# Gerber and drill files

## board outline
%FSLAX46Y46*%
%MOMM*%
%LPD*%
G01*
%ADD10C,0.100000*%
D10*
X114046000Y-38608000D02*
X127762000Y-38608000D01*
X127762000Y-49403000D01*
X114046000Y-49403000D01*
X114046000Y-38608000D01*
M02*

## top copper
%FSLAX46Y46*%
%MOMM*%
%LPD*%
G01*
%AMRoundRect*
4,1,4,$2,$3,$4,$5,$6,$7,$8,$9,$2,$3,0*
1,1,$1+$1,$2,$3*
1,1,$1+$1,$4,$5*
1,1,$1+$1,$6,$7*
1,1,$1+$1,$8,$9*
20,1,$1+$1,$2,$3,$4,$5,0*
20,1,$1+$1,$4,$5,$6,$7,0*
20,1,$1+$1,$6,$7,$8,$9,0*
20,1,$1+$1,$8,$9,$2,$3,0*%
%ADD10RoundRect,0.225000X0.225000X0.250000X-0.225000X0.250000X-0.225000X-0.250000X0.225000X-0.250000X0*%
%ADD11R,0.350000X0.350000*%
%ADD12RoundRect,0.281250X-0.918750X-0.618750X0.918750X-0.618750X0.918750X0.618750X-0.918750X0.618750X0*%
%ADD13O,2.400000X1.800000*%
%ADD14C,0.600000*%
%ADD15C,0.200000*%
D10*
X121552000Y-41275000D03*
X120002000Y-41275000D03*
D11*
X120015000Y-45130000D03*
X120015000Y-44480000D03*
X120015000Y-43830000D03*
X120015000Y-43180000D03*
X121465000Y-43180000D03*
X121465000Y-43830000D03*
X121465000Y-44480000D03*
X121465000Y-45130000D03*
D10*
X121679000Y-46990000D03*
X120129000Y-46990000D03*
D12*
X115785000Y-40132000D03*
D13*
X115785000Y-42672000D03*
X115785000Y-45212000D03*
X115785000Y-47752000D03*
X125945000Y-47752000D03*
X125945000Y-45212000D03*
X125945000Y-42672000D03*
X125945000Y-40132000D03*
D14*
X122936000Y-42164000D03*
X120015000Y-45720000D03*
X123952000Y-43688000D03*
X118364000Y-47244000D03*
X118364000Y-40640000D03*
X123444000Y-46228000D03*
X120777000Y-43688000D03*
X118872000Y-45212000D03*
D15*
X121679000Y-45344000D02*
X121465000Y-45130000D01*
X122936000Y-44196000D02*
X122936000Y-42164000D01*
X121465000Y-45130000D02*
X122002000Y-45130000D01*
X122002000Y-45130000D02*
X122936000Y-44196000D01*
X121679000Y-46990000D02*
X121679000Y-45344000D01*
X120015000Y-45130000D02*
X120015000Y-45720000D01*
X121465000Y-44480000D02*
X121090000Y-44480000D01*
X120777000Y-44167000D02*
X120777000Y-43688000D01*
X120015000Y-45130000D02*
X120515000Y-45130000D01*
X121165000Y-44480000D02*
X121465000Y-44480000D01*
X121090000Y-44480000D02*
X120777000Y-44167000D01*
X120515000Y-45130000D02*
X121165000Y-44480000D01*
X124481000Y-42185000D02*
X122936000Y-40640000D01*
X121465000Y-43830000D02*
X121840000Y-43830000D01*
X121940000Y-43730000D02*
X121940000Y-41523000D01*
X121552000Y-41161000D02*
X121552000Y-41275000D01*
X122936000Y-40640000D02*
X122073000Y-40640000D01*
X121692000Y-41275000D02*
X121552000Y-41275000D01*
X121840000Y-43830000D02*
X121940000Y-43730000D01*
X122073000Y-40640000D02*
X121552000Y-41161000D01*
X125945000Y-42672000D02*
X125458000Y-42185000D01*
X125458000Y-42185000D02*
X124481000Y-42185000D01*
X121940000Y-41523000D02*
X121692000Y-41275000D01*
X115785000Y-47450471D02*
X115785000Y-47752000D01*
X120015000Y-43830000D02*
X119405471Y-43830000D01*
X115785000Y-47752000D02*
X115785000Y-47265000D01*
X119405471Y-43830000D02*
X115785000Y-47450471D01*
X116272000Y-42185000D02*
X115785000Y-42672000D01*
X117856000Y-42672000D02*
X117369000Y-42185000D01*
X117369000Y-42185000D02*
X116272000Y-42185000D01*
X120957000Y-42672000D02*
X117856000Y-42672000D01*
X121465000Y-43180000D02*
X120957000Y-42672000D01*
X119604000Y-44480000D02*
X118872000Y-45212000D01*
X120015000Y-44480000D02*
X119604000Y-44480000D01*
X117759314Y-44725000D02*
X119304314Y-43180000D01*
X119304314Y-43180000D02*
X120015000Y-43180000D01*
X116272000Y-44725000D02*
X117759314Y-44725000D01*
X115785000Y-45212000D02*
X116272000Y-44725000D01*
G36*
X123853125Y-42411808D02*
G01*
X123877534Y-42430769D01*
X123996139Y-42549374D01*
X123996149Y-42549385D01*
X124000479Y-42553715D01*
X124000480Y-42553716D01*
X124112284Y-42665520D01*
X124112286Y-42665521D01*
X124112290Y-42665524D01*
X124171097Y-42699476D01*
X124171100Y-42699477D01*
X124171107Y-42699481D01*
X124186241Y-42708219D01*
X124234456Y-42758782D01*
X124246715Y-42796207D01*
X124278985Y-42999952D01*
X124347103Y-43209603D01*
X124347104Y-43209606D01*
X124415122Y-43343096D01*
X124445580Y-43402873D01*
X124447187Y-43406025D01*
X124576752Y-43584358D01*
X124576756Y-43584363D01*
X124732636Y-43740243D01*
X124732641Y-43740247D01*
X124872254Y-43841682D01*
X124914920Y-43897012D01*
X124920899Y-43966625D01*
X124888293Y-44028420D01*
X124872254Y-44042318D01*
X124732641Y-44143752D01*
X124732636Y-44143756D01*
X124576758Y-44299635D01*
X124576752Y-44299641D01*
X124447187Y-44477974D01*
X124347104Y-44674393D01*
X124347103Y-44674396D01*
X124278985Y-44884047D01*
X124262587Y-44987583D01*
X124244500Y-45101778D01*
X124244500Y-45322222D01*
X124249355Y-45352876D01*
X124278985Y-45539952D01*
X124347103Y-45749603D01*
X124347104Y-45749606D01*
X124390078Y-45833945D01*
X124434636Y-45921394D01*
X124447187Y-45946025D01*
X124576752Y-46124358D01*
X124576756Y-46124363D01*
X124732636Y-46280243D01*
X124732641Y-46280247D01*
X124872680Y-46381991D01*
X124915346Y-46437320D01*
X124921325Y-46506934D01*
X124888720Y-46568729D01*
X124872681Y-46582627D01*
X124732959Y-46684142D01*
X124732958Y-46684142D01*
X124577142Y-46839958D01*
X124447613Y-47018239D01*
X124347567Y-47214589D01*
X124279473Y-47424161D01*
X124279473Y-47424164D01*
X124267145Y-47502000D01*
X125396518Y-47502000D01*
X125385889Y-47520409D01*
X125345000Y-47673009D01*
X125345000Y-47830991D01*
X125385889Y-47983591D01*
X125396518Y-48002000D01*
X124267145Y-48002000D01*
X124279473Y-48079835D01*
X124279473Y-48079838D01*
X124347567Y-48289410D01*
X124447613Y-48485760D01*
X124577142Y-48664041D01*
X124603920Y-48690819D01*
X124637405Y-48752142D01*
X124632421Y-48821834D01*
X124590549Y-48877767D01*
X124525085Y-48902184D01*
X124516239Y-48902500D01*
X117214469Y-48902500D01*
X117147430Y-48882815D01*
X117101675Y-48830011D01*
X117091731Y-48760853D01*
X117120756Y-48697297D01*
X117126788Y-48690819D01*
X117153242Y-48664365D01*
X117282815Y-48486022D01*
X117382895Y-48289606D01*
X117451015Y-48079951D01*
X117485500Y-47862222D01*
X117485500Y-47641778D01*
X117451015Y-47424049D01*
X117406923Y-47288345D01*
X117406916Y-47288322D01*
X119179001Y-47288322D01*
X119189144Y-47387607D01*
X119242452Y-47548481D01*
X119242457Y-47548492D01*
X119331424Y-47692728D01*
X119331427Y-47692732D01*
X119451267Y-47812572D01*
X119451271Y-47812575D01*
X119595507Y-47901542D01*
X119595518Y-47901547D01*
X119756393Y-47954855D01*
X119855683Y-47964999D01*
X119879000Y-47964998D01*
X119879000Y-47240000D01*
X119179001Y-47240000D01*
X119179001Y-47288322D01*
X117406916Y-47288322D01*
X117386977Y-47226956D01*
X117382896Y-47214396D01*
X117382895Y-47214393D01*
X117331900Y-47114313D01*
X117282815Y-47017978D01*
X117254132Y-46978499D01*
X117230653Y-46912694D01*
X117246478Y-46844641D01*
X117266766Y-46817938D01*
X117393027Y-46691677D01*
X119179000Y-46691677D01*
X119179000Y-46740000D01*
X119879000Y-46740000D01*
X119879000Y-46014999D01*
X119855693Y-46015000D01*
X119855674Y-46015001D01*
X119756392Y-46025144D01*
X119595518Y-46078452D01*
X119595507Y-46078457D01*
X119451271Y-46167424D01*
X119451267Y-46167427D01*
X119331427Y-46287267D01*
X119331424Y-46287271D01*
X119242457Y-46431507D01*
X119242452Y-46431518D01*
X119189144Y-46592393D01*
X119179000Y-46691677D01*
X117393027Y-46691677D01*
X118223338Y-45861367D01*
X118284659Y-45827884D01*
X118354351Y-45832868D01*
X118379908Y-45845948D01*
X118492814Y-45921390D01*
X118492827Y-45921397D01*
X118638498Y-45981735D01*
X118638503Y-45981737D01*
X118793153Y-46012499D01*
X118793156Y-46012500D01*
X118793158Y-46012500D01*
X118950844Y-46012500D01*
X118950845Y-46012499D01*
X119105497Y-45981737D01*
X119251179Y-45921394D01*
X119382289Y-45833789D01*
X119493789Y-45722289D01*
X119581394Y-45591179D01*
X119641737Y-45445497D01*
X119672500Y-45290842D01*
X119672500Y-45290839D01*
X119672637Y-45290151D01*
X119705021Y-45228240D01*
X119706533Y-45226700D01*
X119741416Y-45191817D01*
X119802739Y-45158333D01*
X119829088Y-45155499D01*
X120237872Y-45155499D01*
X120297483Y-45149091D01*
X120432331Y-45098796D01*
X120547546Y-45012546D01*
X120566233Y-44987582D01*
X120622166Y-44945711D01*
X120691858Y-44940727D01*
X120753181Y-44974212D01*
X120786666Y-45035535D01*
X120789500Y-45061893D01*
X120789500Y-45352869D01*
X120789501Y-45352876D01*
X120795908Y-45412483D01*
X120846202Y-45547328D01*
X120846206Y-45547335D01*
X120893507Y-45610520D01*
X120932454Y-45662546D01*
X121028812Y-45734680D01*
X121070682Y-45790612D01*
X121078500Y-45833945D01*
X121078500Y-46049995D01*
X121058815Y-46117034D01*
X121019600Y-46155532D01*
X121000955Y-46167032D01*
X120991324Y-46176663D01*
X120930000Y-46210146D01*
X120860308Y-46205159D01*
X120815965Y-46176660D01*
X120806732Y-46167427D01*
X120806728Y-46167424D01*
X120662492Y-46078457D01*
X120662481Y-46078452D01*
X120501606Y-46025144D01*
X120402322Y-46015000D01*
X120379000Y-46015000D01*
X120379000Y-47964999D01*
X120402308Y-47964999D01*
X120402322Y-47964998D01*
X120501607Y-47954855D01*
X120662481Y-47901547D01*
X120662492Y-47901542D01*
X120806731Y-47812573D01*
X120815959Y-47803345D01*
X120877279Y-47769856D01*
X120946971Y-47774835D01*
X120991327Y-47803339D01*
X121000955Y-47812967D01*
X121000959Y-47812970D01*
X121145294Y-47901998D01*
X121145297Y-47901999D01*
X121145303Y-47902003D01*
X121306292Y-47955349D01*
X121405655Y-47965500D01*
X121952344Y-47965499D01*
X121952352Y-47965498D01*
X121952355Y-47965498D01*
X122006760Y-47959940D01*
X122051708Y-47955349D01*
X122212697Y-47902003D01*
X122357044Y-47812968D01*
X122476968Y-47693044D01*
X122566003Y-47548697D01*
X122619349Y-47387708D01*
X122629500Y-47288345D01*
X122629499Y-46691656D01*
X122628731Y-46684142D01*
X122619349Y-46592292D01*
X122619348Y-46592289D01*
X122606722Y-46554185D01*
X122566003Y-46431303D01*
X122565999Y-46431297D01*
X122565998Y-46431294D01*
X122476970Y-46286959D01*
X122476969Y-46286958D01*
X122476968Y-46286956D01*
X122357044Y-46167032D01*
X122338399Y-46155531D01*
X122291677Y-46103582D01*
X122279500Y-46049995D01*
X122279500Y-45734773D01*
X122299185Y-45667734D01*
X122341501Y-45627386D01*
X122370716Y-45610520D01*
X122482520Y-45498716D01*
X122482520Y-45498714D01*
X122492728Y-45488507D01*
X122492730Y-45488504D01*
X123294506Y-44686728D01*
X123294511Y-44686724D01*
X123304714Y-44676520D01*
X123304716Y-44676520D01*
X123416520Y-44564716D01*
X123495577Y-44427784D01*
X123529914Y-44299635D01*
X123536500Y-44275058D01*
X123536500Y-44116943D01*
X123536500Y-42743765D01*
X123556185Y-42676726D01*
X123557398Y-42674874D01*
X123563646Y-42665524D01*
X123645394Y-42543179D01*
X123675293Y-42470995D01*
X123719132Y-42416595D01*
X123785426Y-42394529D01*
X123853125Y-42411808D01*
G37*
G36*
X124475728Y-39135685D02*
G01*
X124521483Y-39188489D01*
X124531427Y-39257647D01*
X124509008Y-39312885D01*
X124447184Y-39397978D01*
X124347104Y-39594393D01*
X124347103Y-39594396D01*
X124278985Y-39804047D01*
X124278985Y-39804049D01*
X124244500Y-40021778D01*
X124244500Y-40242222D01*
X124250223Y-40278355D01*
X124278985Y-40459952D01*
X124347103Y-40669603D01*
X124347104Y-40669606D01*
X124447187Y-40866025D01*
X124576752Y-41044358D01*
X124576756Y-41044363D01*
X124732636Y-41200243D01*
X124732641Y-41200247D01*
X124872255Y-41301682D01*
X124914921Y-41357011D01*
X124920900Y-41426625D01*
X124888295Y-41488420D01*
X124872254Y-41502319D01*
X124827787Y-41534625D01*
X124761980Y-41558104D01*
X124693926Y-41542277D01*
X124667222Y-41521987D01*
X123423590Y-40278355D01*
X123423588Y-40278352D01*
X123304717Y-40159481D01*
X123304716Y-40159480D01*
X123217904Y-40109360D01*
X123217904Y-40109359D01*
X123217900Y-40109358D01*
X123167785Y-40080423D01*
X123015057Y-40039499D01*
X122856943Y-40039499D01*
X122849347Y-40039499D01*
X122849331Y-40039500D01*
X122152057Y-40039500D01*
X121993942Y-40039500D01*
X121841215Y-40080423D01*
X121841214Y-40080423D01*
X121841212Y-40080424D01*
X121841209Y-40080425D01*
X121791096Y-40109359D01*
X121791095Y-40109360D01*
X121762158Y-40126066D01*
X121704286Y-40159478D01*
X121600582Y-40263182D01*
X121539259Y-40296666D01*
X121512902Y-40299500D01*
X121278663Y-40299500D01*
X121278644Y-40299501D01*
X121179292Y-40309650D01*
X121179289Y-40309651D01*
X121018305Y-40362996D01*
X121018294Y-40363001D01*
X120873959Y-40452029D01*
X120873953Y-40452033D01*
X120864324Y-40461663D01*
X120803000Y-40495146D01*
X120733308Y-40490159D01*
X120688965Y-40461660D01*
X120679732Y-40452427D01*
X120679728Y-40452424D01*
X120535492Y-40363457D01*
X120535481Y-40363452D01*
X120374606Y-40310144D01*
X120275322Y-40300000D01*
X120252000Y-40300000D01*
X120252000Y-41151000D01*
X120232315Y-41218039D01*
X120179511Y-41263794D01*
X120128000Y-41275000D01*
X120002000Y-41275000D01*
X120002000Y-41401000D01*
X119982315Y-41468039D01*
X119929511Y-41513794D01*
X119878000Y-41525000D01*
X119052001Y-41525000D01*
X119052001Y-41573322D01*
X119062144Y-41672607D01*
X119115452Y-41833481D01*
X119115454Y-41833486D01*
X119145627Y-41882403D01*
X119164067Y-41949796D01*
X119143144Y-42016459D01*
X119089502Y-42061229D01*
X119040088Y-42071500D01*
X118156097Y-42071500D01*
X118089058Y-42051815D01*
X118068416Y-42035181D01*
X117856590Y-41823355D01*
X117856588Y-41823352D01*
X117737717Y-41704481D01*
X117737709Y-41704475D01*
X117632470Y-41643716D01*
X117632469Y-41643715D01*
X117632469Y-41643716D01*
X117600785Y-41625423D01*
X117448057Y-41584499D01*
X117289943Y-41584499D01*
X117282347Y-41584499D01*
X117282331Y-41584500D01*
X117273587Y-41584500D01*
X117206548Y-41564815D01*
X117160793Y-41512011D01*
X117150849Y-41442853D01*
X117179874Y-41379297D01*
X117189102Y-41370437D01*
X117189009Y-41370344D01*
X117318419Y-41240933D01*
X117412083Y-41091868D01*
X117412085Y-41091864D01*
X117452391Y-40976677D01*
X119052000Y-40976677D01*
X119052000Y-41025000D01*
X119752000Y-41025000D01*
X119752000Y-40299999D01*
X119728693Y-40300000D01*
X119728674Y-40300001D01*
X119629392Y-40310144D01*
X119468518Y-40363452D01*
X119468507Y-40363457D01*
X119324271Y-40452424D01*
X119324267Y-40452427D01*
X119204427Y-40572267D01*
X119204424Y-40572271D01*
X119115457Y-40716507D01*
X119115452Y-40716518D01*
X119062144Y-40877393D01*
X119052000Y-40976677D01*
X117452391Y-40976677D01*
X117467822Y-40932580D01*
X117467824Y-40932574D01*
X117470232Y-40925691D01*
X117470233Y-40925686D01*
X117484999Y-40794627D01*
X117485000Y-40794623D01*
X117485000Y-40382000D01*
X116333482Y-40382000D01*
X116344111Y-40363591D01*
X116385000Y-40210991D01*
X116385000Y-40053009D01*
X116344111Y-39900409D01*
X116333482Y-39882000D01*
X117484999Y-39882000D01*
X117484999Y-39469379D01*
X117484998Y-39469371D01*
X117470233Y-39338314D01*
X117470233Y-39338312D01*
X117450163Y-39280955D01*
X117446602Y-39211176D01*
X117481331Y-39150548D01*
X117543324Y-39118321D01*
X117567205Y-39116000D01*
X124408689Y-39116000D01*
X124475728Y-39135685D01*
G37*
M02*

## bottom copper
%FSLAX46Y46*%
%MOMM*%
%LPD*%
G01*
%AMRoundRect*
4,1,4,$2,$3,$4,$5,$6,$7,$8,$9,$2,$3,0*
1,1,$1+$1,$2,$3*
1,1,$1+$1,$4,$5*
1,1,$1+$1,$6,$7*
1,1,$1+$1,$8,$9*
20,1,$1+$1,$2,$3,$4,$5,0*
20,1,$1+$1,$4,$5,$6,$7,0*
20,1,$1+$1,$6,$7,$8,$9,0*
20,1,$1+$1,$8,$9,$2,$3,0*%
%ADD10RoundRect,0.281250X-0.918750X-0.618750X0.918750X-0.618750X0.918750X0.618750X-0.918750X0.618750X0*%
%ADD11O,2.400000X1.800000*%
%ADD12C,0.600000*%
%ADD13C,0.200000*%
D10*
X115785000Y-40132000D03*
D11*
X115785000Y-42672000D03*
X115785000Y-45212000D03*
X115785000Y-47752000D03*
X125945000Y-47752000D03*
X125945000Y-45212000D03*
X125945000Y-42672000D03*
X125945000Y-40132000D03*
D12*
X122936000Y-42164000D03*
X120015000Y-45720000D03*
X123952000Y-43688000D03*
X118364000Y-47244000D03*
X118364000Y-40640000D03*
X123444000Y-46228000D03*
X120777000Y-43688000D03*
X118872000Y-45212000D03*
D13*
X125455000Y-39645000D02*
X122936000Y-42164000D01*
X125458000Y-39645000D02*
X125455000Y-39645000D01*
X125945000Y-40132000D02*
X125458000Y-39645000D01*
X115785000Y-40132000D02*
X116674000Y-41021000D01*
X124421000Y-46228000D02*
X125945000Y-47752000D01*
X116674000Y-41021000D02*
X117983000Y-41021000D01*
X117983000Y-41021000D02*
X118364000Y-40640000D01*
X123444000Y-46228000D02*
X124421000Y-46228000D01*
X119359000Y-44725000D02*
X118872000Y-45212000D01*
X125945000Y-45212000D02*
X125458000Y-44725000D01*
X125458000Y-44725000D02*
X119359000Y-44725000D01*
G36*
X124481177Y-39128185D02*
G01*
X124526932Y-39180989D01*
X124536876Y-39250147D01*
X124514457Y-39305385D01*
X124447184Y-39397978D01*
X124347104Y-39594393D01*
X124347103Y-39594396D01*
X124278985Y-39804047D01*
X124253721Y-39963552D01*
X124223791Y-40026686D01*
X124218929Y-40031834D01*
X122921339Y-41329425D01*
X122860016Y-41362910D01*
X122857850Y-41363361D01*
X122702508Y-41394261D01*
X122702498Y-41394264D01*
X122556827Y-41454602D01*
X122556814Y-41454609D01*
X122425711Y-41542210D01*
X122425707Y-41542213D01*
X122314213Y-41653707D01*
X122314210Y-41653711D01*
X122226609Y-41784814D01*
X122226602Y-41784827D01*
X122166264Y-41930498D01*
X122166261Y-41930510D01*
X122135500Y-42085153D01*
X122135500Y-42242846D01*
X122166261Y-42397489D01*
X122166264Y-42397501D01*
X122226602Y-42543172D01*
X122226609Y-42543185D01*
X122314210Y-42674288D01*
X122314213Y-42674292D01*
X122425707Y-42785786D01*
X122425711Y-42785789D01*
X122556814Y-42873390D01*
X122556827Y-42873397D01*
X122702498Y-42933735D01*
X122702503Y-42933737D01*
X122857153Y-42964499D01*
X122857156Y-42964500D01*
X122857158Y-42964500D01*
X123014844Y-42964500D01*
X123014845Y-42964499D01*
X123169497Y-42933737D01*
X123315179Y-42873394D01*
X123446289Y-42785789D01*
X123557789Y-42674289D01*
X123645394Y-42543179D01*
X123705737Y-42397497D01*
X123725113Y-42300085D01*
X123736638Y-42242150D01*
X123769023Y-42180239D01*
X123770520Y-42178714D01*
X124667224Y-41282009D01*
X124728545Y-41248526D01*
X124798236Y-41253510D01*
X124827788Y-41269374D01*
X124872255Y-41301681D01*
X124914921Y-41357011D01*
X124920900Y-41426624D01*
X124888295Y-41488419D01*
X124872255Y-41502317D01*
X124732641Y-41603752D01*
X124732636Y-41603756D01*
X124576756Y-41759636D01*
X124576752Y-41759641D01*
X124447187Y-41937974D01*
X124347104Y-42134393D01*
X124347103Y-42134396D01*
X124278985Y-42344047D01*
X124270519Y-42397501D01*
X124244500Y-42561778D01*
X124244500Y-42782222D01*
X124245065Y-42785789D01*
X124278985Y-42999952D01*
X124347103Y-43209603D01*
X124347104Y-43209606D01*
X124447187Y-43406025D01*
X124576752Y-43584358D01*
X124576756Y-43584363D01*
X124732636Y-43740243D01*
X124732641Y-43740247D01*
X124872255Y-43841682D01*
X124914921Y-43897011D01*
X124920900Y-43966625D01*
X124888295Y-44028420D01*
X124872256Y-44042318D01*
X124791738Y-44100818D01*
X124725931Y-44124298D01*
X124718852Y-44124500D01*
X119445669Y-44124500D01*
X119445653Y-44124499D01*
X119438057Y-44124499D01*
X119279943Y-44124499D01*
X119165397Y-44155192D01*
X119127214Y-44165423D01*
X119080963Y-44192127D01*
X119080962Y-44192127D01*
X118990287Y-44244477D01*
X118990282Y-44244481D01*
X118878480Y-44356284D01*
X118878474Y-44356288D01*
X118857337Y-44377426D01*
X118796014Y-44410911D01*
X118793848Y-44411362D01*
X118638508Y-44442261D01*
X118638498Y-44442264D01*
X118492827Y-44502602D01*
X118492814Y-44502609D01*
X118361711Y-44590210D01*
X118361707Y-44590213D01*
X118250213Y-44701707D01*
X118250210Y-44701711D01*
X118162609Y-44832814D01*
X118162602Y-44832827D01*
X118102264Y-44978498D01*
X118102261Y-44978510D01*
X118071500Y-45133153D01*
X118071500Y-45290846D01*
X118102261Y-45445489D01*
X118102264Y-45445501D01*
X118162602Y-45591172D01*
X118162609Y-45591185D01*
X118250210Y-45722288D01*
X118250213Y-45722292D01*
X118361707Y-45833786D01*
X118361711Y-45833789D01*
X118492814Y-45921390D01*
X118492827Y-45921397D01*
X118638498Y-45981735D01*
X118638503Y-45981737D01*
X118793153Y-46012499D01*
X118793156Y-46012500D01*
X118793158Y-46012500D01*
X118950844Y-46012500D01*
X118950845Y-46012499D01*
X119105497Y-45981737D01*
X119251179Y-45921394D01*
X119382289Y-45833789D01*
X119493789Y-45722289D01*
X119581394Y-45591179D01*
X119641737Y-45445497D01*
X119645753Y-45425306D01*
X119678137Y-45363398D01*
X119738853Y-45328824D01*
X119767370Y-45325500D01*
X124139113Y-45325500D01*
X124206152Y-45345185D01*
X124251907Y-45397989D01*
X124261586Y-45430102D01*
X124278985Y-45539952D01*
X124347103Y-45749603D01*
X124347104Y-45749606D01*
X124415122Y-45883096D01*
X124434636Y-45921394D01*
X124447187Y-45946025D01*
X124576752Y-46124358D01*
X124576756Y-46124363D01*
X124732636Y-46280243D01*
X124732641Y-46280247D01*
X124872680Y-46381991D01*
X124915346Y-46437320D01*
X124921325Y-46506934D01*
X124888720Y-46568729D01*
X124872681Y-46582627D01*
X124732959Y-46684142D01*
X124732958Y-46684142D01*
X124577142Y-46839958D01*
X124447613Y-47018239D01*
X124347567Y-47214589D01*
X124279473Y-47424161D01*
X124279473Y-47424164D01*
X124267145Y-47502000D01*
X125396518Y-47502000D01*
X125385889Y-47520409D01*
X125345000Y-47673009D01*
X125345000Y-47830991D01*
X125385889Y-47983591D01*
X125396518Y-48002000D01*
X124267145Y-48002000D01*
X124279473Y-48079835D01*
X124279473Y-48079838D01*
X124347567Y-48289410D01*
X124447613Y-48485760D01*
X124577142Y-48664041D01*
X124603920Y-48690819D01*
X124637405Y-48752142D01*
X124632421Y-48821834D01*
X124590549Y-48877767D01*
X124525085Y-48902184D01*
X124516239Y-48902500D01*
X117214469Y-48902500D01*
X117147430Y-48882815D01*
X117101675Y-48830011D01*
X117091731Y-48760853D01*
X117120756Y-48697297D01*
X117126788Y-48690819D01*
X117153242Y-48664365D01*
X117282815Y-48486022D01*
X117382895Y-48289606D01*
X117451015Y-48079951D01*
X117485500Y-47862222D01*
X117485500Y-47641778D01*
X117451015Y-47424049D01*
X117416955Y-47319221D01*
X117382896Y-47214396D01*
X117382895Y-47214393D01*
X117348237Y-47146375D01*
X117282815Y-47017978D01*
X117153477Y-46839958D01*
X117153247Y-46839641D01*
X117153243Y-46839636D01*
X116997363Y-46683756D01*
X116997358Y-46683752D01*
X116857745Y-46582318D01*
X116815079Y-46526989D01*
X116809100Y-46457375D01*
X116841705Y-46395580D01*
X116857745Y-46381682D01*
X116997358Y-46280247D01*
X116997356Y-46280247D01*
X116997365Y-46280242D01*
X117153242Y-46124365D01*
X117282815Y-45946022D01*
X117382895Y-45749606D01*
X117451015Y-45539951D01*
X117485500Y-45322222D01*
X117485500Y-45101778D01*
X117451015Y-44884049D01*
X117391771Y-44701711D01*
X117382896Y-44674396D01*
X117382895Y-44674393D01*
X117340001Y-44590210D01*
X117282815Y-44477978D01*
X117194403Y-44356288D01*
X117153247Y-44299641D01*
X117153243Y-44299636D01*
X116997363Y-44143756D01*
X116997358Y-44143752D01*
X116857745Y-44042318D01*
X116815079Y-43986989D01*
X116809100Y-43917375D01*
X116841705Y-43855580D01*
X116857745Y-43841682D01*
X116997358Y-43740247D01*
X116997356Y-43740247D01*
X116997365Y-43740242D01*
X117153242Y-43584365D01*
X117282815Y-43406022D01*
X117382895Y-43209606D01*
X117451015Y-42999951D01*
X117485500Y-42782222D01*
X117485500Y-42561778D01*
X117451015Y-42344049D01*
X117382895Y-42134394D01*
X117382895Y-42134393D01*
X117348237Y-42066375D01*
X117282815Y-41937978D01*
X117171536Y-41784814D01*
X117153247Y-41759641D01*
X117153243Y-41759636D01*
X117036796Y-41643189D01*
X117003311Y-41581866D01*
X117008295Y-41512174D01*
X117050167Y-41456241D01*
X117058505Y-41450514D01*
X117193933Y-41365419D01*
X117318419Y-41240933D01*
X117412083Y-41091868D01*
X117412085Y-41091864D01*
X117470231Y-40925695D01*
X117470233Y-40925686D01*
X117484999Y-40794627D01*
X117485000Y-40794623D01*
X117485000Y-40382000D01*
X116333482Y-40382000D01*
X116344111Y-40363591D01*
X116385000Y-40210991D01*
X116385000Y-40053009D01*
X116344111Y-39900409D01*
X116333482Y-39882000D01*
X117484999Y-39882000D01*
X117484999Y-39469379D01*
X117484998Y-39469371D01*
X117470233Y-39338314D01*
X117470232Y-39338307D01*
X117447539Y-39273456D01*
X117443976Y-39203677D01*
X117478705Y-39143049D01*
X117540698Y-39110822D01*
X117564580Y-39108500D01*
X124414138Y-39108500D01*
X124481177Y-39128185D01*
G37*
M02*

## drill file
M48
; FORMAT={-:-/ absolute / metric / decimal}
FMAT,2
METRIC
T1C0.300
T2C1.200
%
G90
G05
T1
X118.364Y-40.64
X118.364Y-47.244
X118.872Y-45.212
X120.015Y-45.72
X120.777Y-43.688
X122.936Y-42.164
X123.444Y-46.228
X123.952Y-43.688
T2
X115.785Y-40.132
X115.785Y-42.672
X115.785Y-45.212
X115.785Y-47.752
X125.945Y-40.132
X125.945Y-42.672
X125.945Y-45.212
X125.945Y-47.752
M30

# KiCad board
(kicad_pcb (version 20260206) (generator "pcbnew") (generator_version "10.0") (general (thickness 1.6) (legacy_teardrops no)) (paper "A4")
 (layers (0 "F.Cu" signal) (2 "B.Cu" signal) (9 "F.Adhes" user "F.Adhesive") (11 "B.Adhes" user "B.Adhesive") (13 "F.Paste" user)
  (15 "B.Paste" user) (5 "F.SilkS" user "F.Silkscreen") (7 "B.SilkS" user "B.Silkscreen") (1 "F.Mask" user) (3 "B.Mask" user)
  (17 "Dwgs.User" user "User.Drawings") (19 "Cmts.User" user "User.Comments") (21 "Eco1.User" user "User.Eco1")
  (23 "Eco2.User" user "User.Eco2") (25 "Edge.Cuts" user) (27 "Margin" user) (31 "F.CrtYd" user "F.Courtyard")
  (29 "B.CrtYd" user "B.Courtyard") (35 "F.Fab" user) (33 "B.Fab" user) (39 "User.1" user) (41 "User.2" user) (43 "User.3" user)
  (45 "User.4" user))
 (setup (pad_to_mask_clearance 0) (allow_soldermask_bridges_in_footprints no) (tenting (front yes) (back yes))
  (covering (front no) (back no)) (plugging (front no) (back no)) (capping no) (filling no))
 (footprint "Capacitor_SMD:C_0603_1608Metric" (layer "F.Cu") (at 120.777 41.275 180)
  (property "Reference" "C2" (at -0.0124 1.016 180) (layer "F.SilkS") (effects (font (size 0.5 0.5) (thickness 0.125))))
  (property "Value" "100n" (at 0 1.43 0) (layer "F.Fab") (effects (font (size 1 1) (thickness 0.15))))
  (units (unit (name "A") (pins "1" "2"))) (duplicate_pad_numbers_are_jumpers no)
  (pad "1" smd roundrect (at -0.775 0 180) (size 0.9 0.95) (layers "F.Cu" "F.Mask" "F.Paste") (roundrect_rratio 0.25) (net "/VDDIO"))
  (pad "2" smd roundrect (at 0.775 0 180) (size 0.9 0.95) (layers "F.Cu" "F.Mask" "F.Paste") (roundrect_rratio 0.25) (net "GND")))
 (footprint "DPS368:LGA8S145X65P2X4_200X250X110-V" (layer "F.Cu") (at 120.74 44.155 90)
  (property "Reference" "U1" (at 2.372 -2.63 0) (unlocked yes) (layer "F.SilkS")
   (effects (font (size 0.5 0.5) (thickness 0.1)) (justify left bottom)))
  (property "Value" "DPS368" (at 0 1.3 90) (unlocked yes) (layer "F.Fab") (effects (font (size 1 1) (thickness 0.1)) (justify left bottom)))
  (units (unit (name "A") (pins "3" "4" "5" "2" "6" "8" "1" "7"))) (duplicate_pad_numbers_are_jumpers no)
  (pad "1" smd rect (at -0.975 -0.725 90) (size 0.35 0.35) (layers "F.Cu" "F.Mask") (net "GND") (solder_mask_margin 0.1016) (zone_connect 2)
   (thermal_bridge_angle 0))
  (pad "2" smd rect (at -0.325 -0.725 90) (size 0.35 0.35) (layers "F.Cu" "F.Mask") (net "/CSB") (solder_mask_margin 0.1016)
   (zone_connect 2) (thermal_bridge_angle 0))
  (pad "3" smd rect (at 0.325 -0.725 90) (size 0.35 0.35) (layers "F.Cu" "F.Mask") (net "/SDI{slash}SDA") (solder_mask_margin 0.1016)
   (zone_connect 2) (thermal_bridge_angle 0))
  (pad "4" smd rect (at 0.975 -0.725 90) (size 0.35 0.35) (layers "F.Cu" "F.Mask") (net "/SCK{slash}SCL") (solder_mask_margin 0.1016)
   (zone_connect 2) (thermal_bridge_angle 0))
  (pad "5" smd rect (at 0.975 0.725 90) (size 0.35 0.35) (layers "F.Cu" "F.Mask") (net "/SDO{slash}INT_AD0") (solder_mask_margin 0.1016)
   (zone_connect 2) (thermal_bridge_angle 0))
  (pad "6" smd rect (at 0.325 0.725 90) (size 0.35 0.35) (layers "F.Cu" "F.Mask") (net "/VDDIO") (solder_mask_margin 0.1016)
   (zone_connect 2) (thermal_bridge_angle 0))
  (pad "7" smd rect (at -0.325 0.725 90) (size 0.35 0.35) (layers "F.Cu" "F.Mask") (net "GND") (solder_mask_margin 0.1016) (zone_connect 2)
   (thermal_bridge_angle 0))
  (pad "8" smd rect (at -0.975 0.725 90) (size 0.35 0.35) (layers "F.Cu" "F.Mask") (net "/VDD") (solder_mask_margin 0.1016) (zone_connect 2)
   (thermal_bridge_angle 0)))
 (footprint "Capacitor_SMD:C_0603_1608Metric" (layer "F.Cu") (at 120.904 46.99 180)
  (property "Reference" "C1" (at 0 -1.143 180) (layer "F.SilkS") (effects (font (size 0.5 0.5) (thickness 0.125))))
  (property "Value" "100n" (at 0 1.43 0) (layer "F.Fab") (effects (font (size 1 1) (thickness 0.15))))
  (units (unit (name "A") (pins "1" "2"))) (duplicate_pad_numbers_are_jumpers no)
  (pad "1" smd roundrect (at -0.775 0 180) (size 0.9 0.95) (layers "F.Cu" "F.Mask" "F.Paste") (roundrect_rratio 0.25) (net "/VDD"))
  (pad "2" smd roundrect (at 0.775 0 180) (size 0.9 0.95) (layers "F.Cu" "F.Mask" "F.Paste") (roundrect_rratio 0.25) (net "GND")))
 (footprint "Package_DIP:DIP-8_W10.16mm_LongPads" (layer "F.Cu") (at 115.785 40.132)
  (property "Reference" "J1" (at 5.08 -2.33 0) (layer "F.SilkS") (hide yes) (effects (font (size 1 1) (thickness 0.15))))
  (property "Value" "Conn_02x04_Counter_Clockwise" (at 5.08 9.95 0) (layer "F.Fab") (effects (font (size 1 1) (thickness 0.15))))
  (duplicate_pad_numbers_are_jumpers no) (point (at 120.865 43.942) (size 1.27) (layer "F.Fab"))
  (pad "1" thru_hole roundrect (at 0 0) (size 2.4 1.8) (drill 1.2) (layers "*.Cu" "*.Mask") (remove_unused_layers no)
   (roundrect_rratio 0.15625) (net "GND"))
  (pad "2" thru_hole oval (at 0 2.54) (size 2.4 1.8) (drill 1.2) (layers "*.Cu" "*.Mask") (remove_unused_layers no)
   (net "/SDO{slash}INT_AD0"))
  (pad "3" thru_hole oval (at 0 5.08) (size 2.4 1.8) (drill 1.2) (layers "*.Cu" "*.Mask") (remove_unused_layers no) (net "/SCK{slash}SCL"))
  (pad "4" thru_hole oval (at 0 7.62) (size 2.4 1.8) (drill 1.2) (layers "*.Cu" "*.Mask") (remove_unused_layers no) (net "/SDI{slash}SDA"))
  (pad "5" thru_hole oval (at 10.16 7.62) (size 2.4 1.8) (drill 1.2) (layers "*.Cu" "*.Mask") (remove_unused_layers no) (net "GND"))
  (pad "6" thru_hole oval (at 10.16 5.08) (size 2.4 1.8) (drill 1.2) (layers "*.Cu" "*.Mask") (remove_unused_layers no) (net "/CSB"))
  (pad "7" thru_hole oval (at 10.16 2.54) (size 2.4 1.8) (drill 1.2) (layers "*.Cu" "*.Mask") (remove_unused_layers no) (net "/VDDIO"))
  (pad "8" thru_hole oval (at 10.16 0) (size 2.4 1.8) (drill 1.2) (layers "*.Cu" "*.Mask") (remove_unused_layers no) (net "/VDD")))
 (gr_rect (start 114.046 38.608) (end 127.762 49.403) (stroke (width 0.1) (type solid)) (fill no) (layer "Edge.Cuts"))
 (segment (start 121.679 45.344) (end 121.465 45.13) (width 0.2) (layer "F.Cu") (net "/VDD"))
 (segment (start 122.936 44.196) (end 122.936 42.164) (width 0.2) (layer "F.Cu") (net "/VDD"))
 (segment (start 121.465 45.13) (end 122.002 45.13) (width 0.2) (layer "F.Cu") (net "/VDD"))
 (segment (start 122.002 45.13) (end 122.936 44.196) (width 0.2) (layer "F.Cu") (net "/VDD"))
 (segment (start 121.679 46.99) (end 121.679 45.344) (width 0.2) (layer "F.Cu") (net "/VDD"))
 (via (at 122.936 42.164) (size 0.6) (drill 0.3) (layers "F.Cu" "B.Cu") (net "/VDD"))
 (segment (start 125.455 39.645) (end 122.936 42.164) (width 0.2) (layer "B.Cu") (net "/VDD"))
 (segment (start 125.458 39.645) (end 125.455 39.645) (width 0.2) (layer "B.Cu") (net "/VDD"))
 (segment (start 125.945 40.132) (end 125.458 39.645) (width 0.2) (layer "B.Cu") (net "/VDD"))
 (segment (start 120.015 45.13) (end 120.015 45.72) (width 0.2) (layer "F.Cu") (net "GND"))
 (segment (start 121.465 44.48) (end 121.09 44.48) (width 0.2) (layer "F.Cu") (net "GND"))
 (segment (start 120.777 44.167) (end 120.777 43.688) (width 0.2) (layer "F.Cu") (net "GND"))
 (segment (start 120.015 45.13) (end 120.515 45.13) (width 0.2) (layer "F.Cu") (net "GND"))
 (segment (start 121.165 44.48) (end 121.465 44.48) (width 0.2) (layer "F.Cu") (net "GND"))
 (segment (start 121.09 44.48) (end 120.777 44.167) (width 0.2) (layer "F.Cu") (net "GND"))
 (segment (start 120.515 45.13) (end 121.165 44.48) (width 0.2) (layer "F.Cu") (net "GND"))
 (via (at 120.015 45.72) (size 0.6) (drill 0.3) (layers "F.Cu" "B.Cu") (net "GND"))
 (via (at 123.952 43.688) (size 0.6) (drill 0.3) (layers "F.Cu" "B.Cu") (free yes) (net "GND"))
 (via (at 118.364 47.244) (size 0.6) (drill 0.3) (layers "F.Cu" "B.Cu") (free yes) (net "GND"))
 (via (at 118.364 40.64) (size 0.6) (drill 0.3) (layers "F.Cu" "B.Cu") (free yes) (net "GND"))
 (via (at 123.444 46.228) (size 0.6) (drill 0.3) (layers "F.Cu" "B.Cu") (free yes) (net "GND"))
 (via (at 120.777 43.688) (size 0.6) (drill 0.3) (layers "F.Cu" "B.Cu") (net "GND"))
 (segment (start 115.785 40.132) (end 116.674 41.021) (width 0.2) (layer "B.Cu") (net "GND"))
 (segment (start 124.421 46.228) (end 125.945 47.752) (width 0.2) (layer "B.Cu") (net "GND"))
 (segment (start 116.674 41.021) (end 117.983 41.021) (width 0.2) (layer "B.Cu") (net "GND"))
 (segment (start 117.983 41.021) (end 118.364 40.64) (width 0.2) (layer "B.Cu") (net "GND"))
 (segment (start 123.444 46.228) (end 124.421 46.228) (width 0.2) (layer "B.Cu") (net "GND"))
 (segment (start 124.481 42.185) (end 122.936 40.64) (width 0.2) (layer "F.Cu") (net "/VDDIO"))
 (segment (start 121.465 43.83) (end 121.84 43.83) (width 0.2) (layer "F.Cu") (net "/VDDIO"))
 (segment (start 121.94 43.73) (end 121.94 41.523) (width 0.2) (layer "F.Cu") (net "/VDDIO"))
 (segment (start 121.552 41.161) (end 121.552 41.275) (width 0.2) (layer "F.Cu") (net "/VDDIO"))
 (segment (start 122.936 40.64) (end 122.073 40.64) (width 0.2) (layer "F.Cu") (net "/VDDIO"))
 (segment (start 121.692 41.275) (end 121.552 41.275) (width 0.2) (layer "F.Cu") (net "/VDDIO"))
 (segment (start 121.84 43.83) (end 121.94 43.73) (width 0.2) (layer "F.Cu") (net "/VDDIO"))
 (segment (start 122.073 40.64) (end 121.552 41.161) (width 0.2) (layer "F.Cu") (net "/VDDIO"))
 (segment (start 125.945 42.672) (end 125.458 42.185) (width 0.2) (layer "F.Cu") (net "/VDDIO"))
 (segment (start 125.458 42.185) (end 124.481 42.185) (width 0.2) (layer "F.Cu") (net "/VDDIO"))
 (segment (start 121.94 41.523) (end 121.692 41.275) (width 0.2) (layer "F.Cu") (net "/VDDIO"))
 (segment (start 115.785 47.450471) (end 115.785 47.752) (width 0.2) (layer "F.Cu") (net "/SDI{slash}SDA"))
 (segment (start 120.015 43.83) (end 119.405471 43.83) (width 0.2) (layer "F.Cu") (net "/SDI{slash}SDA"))
 (segment (start 115.785 47.752) (end 115.785 47.265) (width 0.2) (layer "F.Cu") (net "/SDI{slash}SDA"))
 (segment (start 119.405471 43.83) (end 115.785 47.450471) (width 0.2) (layer "F.Cu") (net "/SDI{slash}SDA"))
 (segment (start 116.272 42.185) (end 115.785 42.672) (width 0.2) (layer "F.Cu") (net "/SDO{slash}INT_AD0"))
 (segment (start 117.856 42.672) (end 117.369 42.185) (width 0.2) (layer "F.Cu") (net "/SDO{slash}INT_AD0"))
 (segment (start 117.369 42.185) (end 116.272 42.185) (width 0.2) (layer "F.Cu") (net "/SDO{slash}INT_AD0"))
 (segment (start 120.957 42.672) (end 117.856 42.672) (width 0.2) (layer "F.Cu") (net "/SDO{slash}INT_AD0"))
 (segment (start 121.465 43.18) (end 120.957 42.672) (width 0.2) (layer "F.Cu") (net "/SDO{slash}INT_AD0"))
 (segment (start 119.604 44.48) (end 118.872 45.212) (width 0.2) (layer "F.Cu") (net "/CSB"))
 (segment (start 120.015 44.48) (end 119.604 44.48) (width 0.2) (layer "F.Cu") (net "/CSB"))
 (via (at 118.872 45.212) (size 0.6) (drill 0.3) (layers "F.Cu" "B.Cu") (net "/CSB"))
 (segment (start 119.359 44.725) (end 118.872 45.212) (width 0.2) (layer "B.Cu") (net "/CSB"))
 (segment (start 125.945 45.212) (end 125.458 44.725) (width 0.2) (layer "B.Cu") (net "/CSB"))
 (segment (start 125.458 44.725) (end 119.359 44.725) (width 0.2) (layer "B.Cu") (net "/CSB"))
 (segment (start 117.759314 44.725) (end 119.304314 43.18) (width 0.2) (layer "F.Cu") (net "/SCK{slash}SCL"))
 (segment (start 119.304314 43.18) (end 120.015 43.18) (width 0.2) (layer "F.Cu") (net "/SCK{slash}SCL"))
 (segment (start 116.272 44.725) (end 117.759314 44.725) (width 0.2) (layer "F.Cu") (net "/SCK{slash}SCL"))
 (segment (start 115.785 45.212) (end 116.272 44.725) (width 0.2) (layer "F.Cu") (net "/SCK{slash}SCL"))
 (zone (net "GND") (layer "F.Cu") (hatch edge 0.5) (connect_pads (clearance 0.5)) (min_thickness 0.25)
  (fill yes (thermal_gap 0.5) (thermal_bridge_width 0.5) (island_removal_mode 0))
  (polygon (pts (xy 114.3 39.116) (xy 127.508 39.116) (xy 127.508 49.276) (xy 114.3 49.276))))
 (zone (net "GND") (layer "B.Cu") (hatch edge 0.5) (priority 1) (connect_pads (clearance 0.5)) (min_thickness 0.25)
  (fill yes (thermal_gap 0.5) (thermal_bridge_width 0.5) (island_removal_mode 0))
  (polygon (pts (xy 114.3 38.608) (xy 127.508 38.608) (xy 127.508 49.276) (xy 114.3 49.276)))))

